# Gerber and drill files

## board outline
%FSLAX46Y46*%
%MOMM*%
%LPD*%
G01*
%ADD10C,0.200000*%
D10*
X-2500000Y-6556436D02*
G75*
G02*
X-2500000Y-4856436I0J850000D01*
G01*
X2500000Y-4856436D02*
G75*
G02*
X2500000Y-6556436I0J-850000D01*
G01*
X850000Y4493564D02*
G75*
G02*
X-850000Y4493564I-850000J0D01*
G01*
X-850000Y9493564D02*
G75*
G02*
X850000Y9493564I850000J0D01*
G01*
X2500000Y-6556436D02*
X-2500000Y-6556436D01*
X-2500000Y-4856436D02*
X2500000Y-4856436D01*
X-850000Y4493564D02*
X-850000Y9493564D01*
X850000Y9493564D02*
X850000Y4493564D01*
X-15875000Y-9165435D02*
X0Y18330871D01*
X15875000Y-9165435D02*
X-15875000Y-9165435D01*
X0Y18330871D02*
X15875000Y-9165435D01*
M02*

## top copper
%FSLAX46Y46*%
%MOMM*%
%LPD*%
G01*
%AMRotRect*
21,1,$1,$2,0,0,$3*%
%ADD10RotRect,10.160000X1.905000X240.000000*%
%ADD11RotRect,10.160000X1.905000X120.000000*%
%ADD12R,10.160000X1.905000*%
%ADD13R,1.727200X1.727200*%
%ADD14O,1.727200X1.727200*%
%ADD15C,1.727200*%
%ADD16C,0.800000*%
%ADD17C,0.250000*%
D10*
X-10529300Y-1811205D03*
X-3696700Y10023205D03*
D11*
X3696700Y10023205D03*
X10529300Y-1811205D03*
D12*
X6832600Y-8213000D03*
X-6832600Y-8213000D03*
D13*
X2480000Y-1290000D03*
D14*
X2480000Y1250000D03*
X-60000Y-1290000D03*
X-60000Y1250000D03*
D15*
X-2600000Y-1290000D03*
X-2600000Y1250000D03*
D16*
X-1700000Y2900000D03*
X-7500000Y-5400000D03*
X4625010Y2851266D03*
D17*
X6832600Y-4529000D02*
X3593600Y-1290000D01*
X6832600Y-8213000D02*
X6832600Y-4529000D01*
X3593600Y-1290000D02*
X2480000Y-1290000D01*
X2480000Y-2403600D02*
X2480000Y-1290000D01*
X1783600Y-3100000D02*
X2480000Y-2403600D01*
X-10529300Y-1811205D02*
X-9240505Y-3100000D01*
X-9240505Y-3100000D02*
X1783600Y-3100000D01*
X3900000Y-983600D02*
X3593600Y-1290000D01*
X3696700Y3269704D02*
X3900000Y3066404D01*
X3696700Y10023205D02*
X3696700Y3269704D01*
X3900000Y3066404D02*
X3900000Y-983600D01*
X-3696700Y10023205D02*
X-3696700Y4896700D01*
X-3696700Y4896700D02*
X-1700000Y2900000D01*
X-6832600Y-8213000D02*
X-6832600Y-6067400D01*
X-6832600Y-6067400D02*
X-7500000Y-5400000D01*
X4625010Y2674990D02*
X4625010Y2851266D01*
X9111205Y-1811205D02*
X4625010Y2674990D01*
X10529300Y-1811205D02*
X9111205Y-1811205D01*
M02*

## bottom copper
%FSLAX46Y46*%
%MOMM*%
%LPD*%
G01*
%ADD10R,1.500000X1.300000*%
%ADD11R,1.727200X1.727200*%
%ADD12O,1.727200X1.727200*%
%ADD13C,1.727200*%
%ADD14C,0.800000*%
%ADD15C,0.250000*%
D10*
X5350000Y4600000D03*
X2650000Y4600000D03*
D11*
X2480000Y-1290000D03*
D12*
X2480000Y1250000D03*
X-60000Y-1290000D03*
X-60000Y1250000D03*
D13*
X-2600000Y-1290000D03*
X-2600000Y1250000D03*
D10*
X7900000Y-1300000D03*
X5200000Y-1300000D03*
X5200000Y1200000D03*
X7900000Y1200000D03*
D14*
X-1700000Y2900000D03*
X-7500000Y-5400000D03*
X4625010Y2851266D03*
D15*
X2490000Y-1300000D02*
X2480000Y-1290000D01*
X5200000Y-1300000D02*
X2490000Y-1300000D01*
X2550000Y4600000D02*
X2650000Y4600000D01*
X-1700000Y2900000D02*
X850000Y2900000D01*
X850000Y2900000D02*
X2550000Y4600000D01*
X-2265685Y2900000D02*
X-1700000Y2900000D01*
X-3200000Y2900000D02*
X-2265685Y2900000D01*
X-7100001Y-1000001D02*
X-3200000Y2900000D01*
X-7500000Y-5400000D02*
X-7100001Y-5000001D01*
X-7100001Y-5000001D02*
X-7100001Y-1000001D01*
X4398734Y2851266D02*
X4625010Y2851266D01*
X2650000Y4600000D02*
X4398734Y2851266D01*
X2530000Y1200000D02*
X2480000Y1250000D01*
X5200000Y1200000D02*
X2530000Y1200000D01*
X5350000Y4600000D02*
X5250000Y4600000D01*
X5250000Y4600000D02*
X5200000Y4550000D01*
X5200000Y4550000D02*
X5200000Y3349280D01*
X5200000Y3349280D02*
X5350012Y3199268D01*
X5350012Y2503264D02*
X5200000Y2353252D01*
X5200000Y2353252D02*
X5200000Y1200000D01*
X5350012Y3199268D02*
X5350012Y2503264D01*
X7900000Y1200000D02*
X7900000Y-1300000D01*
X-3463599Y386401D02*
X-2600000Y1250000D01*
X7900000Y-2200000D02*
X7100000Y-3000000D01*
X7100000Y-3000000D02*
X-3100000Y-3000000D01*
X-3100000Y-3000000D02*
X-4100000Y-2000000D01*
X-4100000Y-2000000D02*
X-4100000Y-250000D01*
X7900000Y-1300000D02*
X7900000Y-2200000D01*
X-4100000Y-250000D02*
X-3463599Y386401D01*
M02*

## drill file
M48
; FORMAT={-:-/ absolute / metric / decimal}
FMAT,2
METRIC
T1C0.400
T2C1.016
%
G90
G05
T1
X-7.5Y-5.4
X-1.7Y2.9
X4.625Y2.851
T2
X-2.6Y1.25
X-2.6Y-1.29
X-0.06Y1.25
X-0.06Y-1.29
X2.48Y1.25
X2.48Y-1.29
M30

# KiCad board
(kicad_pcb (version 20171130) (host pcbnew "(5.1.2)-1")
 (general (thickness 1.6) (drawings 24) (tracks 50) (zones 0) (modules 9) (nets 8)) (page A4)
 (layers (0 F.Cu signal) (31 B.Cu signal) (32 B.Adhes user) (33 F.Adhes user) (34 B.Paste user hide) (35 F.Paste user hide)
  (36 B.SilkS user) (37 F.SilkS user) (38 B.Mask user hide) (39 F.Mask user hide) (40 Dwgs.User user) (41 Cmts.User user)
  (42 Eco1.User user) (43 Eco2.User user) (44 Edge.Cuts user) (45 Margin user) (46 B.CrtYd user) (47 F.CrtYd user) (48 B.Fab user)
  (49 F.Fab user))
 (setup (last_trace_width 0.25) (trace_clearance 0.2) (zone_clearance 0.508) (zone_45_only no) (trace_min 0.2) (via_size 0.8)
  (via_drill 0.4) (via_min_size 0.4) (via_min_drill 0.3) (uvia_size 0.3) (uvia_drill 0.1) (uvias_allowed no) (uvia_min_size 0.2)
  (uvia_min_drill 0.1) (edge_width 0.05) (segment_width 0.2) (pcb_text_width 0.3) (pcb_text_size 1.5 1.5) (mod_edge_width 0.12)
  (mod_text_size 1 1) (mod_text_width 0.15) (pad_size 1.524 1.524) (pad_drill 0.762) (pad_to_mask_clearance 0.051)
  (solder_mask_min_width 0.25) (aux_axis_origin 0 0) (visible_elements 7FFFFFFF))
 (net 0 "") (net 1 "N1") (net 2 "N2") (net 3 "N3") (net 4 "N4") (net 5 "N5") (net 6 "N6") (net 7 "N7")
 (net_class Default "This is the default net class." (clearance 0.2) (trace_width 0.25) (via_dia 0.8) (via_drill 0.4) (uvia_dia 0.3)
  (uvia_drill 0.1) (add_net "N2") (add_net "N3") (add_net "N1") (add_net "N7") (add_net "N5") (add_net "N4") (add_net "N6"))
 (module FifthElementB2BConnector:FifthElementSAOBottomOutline (layer F.Cu) (at 0 0)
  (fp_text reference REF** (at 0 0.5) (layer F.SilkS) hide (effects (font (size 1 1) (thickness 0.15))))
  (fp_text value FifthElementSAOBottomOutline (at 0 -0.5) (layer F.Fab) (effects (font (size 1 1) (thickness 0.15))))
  (fp_arc (start -2.5 5.706436) (end -2.5 4.856436) (angle -180) (layer Edge.Cuts) (width 0.2))
  (fp_arc (start 2.5 5.706436) (end 2.5 6.556436) (angle -180) (layer Edge.Cuts) (width 0.2))
  (fp_arc (start 0 -4.493564) (end -0.85 -4.493564) (angle -180) (layer Edge.Cuts) (width 0.2))
  (fp_arc (start 0 -9.493564) (end 0.85 -9.493564) (angle -180) (layer Edge.Cuts) (width 0.2))
  (fp_line (start 2.5 6.556436) (end -2.5 6.556436) (layer Edge.Cuts) (width 0.2))
  (fp_line (start -2.5 4.856436) (end 2.5 4.856436) (layer Edge.Cuts) (width 0.2))
  (fp_line (start -0.85 -4.493564) (end -0.85 -9.493564) (layer Edge.Cuts) (width 0.2))
  (fp_line (start 0.85 -9.493564) (end 0.85 -4.493564) (layer Edge.Cuts) (width 0.2))
  (fp_line (start -15.875 9.165435) (end 0 -18.330871) (layer Edge.Cuts) (width 0.2))
  (fp_line (start 15.875 9.165435) (end -15.875 9.165435) (layer Edge.Cuts) (width 0.2))
  (fp_line (start 0 -18.330871) (end 15.875 9.165435) (layer Edge.Cuts) (width 0.2)))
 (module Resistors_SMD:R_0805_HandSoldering (layer B.Cu) (at 4 -4.6 180)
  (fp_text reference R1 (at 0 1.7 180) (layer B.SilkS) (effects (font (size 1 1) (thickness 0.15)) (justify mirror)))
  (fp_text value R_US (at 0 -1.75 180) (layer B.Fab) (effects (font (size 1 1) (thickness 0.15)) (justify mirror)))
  (pad 1 smd rect (at -1.35 0 180) (size 1.5 1.3) (layers B.Cu B.Paste B.Mask) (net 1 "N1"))
  (pad 2 smd rect (at 1.35 0 180) (size 1.5 1.3) (layers B.Cu B.Paste B.Mask) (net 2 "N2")))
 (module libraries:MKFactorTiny (layer B.Cu) (at -6.9 0.8 180)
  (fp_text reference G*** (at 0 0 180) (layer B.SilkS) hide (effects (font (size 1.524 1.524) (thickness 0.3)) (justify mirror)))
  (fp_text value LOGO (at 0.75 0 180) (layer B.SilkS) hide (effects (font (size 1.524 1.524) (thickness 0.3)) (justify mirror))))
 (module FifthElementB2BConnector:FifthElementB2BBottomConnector (layer F.Cu) (at -7.113 -4.106 240)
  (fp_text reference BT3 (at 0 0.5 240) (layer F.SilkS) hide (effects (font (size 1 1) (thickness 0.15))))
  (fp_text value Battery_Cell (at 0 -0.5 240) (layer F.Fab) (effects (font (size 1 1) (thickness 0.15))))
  (pad 2 smd rect (at 6.8326 0 240) (size 10.16 1.905) (layers F.Cu F.Paste F.Mask) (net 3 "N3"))
  (pad 1 smd rect (at -6.8326 0 240) (size 10.16 1.905) (layers F.Cu F.Paste F.Mask) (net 2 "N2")))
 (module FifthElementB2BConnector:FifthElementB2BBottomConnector (layer F.Cu) (at 7.113 -4.106 120)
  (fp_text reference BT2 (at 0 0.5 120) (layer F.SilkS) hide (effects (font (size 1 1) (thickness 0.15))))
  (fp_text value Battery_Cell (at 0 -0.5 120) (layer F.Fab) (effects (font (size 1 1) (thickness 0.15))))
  (pad 2 smd rect (at 6.8326 0 120) (size 10.16 1.905) (layers F.Cu F.Paste F.Mask) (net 3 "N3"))
  (pad 1 smd rect (at -6.8326 0 120) (size 10.16 1.905) (layers F.Cu F.Paste F.Mask) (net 2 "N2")))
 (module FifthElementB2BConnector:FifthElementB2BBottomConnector (layer F.Cu) (at 0 8.213)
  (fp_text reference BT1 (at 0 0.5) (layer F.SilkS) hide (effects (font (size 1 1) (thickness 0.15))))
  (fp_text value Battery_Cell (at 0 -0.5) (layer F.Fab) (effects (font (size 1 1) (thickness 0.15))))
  (pad 2 smd rect (at 6.8326 0) (size 10.16 1.905) (layers F.Cu F.Paste F.Mask) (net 3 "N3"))
  (pad 1 smd rect (at -6.8326 0) (size 10.16 1.905) (layers F.Cu F.Paste F.Mask) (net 2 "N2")))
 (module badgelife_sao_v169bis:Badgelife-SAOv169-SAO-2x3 (layer B.Cu) (at 0 0 180)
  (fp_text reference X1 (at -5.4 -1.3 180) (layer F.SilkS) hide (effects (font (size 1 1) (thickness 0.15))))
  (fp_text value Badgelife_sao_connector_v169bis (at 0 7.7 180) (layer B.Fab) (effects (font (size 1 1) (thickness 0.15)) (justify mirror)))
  (pad 2 thru_hole rect (at -2.48 -1.29 270) (size 1.7272 1.7272) (drill 1.016) (layers *.Cu *.Mask) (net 3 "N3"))
  (pad 1 thru_hole oval (at -2.48 1.25 270) (size 1.7272 1.7272) (drill 1.016) (layers *.Cu *.Mask) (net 1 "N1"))
  (pad 4 thru_hole oval (at 0.06 -1.29 270) (size 1.7272 1.7272) (drill 1.016) (layers *.Cu *.Mask) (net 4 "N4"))
  (pad 3 thru_hole oval (at 0.06 1.25 270) (size 1.7272 1.7272) (drill 1.016) (layers *.Cu *.Mask) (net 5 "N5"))
  (pad 6 thru_hole circle (at 2.6 -1.29 270) (size 1.7272 1.7272) (drill 1.016) (layers *.Cu *.Mask) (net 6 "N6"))
  (pad 5 thru_hole circle (at 2.6 1.25 270) (size 1.7272 1.7272) (drill 1.016) (layers *.Cu *.Mask) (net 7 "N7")))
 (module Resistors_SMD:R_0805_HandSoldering (layer B.Cu) (at 6.55 1.3 180)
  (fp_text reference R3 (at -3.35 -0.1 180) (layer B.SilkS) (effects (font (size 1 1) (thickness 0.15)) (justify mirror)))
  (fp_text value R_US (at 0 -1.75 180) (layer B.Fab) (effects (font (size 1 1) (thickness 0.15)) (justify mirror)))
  (pad 1 smd rect (at -1.35 0 180) (size 1.5 1.3) (layers B.Cu B.Paste B.Mask) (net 7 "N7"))
  (pad 2 smd rect (at 1.35 0 180) (size 1.5 1.3) (layers B.Cu B.Paste B.Mask) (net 3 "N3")))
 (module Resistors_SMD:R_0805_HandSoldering (layer B.Cu) (at 6.55 -1.2)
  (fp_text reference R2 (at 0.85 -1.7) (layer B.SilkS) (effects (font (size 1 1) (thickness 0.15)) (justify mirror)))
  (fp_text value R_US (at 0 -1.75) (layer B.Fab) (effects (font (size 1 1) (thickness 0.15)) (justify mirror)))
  (pad 1 smd rect (at -1.35 0) (size 1.5 1.3) (layers B.Cu B.Paste B.Mask) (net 1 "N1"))
  (pad 2 smd rect (at 1.35 0) (size 1.5 1.3) (layers B.Cu B.Paste B.Mask) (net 7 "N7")))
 (segment (start 2.49 1.3) (end 2.48 1.29) (width 0.25) (layer B.Cu) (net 3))
 (segment (start 5.2 1.3) (end 2.49 1.3) (width 0.25) (layer B.Cu) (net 3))
 (segment (start 6.8326 4.529) (end 3.5936 1.29) (width 0.25) (layer F.Cu) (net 3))
 (segment (start 6.8326 8.213) (end 6.8326 4.529) (width 0.25) (layer F.Cu) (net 3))
 (segment (start 3.5936 1.29) (end 2.48 1.29) (width 0.25) (layer F.Cu) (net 3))
 (segment (start 2.48 2.4036) (end 2.48 1.29) (width 0.25) (layer F.Cu) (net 3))
 (segment (start 1.7836 3.1) (end 2.48 2.4036) (width 0.25) (layer F.Cu) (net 3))
 (segment (start -10.5293 1.811205) (end -9.240505 3.1) (width 0.25) (layer F.Cu) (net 3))
 (segment (start -9.240505 3.1) (end 1.7836 3.1) (width 0.25) (layer F.Cu) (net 3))
 (segment (start 3.9 0.9836) (end 3.5936 1.29) (width 0.25) (layer F.Cu) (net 3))
 (segment (start 3.6967 -3.269704) (end 3.9 -3.066404) (width 0.25) (layer F.Cu) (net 3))
 (segment (start 3.6967 -10.023205) (end 3.6967 -3.269704) (width 0.25) (layer F.Cu) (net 3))
 (segment (start 3.9 -3.066404) (end 3.9 0.9836) (width 0.25) (layer F.Cu) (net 3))
 (via (at -1.7 -2.9) (size 0.8) (drill 0.4) (layers F.Cu B.Cu) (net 2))
 (segment (start -3.6967 -10.023205) (end -3.6967 -4.8967) (width 0.25) (layer F.Cu) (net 2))
 (segment (start -3.6967 -4.8967) (end -1.7 -2.9) (width 0.25) (layer F.Cu) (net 2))
 (via (at -7.5 5.4) (size 0.8) (drill 0.4) (layers F.Cu B.Cu) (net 2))
 (segment (start -6.8326 8.213) (end -6.8326 6.0674) (width 0.25) (layer F.Cu) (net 2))
 (segment (start -6.8326 6.0674) (end -7.5 5.4) (width 0.25) (layer F.Cu) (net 2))
 (segment (start 2.55 -4.6) (end 2.65 -4.6) (width 0.25) (layer B.Cu) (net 2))
 (segment (start -1.7 -2.9) (end 0.85 -2.9) (width 0.25) (layer B.Cu) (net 2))
 (segment (start 0.85 -2.9) (end 2.55 -4.6) (width 0.25) (layer B.Cu) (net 2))
 (segment (start -2.265685 -2.9) (end -1.7 -2.9) (width 0.25) (layer B.Cu) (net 2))
 (segment (start -3.2 -2.9) (end -2.265685 -2.9) (width 0.25) (layer B.Cu) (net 2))
 (segment (start -7.100001 1.000001) (end -3.2 -2.9) (width 0.25) (layer B.Cu) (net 2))
 (segment (start -7.5 5.4) (end -7.100001 5.000001) (width 0.25) (layer B.Cu) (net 2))
 (segment (start -7.100001 5.000001) (end -7.100001 1.000001) (width 0.25) (layer B.Cu) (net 2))
 (via (at 4.62501 -2.851266) (size 0.8) (drill 0.4) (layers F.Cu B.Cu) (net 2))
 (segment (start 4.62501 -2.67499) (end 4.62501 -2.851266) (width 0.25) (layer F.Cu) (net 2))
 (segment (start 4.398734 -2.851266) (end 4.62501 -2.851266) (width 0.25) (layer B.Cu) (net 2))
 (segment (start 2.65 -4.6) (end 4.398734 -2.851266) (width 0.25) (layer B.Cu) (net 2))
 (segment (start 9.111205 1.811205) (end 4.62501 -2.67499) (width 0.25) (layer F.Cu) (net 2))
 (segment (start 10.5293 1.811205) (end 9.111205 1.811205) (width 0.25) (layer F.Cu) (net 2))
 (segment (start 2.53 -1.2) (end 2.48 -1.25) (width 0.25) (layer B.Cu) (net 1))
 (segment (start 5.2 -1.2) (end 2.53 -1.2) (width 0.25) (layer B.Cu) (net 1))
 (segment (start 5.35 -4.6) (end 5.25 -4.6) (width 0.25) (layer B.Cu) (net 1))
 (segment (start 5.25 -4.6) (end 5.2 -4.55) (width 0.25) (layer B.Cu) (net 1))
 (segment (start 5.2 -4.55) (end 5.2 -3.34928) (width 0.25) (layer B.Cu) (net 1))
 (segment (start 5.2 -3.34928) (end 5.350012 -3.199268) (width 0.25) (layer B.Cu) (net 1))
 (segment (start 5.350012 -2.503264) (end 5.2 -2.353252) (width 0.25) (layer B.Cu) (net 1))
 (segment (start 5.2 -2.353252) (end 5.2 -1.2) (width 0.25) (layer B.Cu) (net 1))
 (segment (start 5.350012 -3.199268) (end 5.350012 -2.503264) (width 0.25) (layer B.Cu) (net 1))
 (segment (start 7.9 -1.2) (end 7.9 1.3) (width 0.25) (layer B.Cu) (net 7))
 (segment (start -3.463599 -0.386401) (end -2.6 -1.25) (width 0.25) (layer B.Cu) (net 7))
 (segment (start 7.9 2.2) (end 7.1 3) (width 0.25) (layer B.Cu) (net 7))
 (segment (start 7.1 3) (end -3.1 3) (width 0.25) (layer B.Cu) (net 7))
 (segment (start -3.1 3) (end -4.1 2) (width 0.25) (layer B.Cu) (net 7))
 (segment (start -4.1 2) (end -4.1 0.25) (width 0.25) (layer B.Cu) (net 7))
 (segment (start 7.9 1.3) (end 7.9 2.2) (width 0.25) (layer B.Cu) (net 7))
 (segment (start -4.1 0.25) (end -3.463599 -0.386401) (width 0.25) (layer B.Cu) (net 7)))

